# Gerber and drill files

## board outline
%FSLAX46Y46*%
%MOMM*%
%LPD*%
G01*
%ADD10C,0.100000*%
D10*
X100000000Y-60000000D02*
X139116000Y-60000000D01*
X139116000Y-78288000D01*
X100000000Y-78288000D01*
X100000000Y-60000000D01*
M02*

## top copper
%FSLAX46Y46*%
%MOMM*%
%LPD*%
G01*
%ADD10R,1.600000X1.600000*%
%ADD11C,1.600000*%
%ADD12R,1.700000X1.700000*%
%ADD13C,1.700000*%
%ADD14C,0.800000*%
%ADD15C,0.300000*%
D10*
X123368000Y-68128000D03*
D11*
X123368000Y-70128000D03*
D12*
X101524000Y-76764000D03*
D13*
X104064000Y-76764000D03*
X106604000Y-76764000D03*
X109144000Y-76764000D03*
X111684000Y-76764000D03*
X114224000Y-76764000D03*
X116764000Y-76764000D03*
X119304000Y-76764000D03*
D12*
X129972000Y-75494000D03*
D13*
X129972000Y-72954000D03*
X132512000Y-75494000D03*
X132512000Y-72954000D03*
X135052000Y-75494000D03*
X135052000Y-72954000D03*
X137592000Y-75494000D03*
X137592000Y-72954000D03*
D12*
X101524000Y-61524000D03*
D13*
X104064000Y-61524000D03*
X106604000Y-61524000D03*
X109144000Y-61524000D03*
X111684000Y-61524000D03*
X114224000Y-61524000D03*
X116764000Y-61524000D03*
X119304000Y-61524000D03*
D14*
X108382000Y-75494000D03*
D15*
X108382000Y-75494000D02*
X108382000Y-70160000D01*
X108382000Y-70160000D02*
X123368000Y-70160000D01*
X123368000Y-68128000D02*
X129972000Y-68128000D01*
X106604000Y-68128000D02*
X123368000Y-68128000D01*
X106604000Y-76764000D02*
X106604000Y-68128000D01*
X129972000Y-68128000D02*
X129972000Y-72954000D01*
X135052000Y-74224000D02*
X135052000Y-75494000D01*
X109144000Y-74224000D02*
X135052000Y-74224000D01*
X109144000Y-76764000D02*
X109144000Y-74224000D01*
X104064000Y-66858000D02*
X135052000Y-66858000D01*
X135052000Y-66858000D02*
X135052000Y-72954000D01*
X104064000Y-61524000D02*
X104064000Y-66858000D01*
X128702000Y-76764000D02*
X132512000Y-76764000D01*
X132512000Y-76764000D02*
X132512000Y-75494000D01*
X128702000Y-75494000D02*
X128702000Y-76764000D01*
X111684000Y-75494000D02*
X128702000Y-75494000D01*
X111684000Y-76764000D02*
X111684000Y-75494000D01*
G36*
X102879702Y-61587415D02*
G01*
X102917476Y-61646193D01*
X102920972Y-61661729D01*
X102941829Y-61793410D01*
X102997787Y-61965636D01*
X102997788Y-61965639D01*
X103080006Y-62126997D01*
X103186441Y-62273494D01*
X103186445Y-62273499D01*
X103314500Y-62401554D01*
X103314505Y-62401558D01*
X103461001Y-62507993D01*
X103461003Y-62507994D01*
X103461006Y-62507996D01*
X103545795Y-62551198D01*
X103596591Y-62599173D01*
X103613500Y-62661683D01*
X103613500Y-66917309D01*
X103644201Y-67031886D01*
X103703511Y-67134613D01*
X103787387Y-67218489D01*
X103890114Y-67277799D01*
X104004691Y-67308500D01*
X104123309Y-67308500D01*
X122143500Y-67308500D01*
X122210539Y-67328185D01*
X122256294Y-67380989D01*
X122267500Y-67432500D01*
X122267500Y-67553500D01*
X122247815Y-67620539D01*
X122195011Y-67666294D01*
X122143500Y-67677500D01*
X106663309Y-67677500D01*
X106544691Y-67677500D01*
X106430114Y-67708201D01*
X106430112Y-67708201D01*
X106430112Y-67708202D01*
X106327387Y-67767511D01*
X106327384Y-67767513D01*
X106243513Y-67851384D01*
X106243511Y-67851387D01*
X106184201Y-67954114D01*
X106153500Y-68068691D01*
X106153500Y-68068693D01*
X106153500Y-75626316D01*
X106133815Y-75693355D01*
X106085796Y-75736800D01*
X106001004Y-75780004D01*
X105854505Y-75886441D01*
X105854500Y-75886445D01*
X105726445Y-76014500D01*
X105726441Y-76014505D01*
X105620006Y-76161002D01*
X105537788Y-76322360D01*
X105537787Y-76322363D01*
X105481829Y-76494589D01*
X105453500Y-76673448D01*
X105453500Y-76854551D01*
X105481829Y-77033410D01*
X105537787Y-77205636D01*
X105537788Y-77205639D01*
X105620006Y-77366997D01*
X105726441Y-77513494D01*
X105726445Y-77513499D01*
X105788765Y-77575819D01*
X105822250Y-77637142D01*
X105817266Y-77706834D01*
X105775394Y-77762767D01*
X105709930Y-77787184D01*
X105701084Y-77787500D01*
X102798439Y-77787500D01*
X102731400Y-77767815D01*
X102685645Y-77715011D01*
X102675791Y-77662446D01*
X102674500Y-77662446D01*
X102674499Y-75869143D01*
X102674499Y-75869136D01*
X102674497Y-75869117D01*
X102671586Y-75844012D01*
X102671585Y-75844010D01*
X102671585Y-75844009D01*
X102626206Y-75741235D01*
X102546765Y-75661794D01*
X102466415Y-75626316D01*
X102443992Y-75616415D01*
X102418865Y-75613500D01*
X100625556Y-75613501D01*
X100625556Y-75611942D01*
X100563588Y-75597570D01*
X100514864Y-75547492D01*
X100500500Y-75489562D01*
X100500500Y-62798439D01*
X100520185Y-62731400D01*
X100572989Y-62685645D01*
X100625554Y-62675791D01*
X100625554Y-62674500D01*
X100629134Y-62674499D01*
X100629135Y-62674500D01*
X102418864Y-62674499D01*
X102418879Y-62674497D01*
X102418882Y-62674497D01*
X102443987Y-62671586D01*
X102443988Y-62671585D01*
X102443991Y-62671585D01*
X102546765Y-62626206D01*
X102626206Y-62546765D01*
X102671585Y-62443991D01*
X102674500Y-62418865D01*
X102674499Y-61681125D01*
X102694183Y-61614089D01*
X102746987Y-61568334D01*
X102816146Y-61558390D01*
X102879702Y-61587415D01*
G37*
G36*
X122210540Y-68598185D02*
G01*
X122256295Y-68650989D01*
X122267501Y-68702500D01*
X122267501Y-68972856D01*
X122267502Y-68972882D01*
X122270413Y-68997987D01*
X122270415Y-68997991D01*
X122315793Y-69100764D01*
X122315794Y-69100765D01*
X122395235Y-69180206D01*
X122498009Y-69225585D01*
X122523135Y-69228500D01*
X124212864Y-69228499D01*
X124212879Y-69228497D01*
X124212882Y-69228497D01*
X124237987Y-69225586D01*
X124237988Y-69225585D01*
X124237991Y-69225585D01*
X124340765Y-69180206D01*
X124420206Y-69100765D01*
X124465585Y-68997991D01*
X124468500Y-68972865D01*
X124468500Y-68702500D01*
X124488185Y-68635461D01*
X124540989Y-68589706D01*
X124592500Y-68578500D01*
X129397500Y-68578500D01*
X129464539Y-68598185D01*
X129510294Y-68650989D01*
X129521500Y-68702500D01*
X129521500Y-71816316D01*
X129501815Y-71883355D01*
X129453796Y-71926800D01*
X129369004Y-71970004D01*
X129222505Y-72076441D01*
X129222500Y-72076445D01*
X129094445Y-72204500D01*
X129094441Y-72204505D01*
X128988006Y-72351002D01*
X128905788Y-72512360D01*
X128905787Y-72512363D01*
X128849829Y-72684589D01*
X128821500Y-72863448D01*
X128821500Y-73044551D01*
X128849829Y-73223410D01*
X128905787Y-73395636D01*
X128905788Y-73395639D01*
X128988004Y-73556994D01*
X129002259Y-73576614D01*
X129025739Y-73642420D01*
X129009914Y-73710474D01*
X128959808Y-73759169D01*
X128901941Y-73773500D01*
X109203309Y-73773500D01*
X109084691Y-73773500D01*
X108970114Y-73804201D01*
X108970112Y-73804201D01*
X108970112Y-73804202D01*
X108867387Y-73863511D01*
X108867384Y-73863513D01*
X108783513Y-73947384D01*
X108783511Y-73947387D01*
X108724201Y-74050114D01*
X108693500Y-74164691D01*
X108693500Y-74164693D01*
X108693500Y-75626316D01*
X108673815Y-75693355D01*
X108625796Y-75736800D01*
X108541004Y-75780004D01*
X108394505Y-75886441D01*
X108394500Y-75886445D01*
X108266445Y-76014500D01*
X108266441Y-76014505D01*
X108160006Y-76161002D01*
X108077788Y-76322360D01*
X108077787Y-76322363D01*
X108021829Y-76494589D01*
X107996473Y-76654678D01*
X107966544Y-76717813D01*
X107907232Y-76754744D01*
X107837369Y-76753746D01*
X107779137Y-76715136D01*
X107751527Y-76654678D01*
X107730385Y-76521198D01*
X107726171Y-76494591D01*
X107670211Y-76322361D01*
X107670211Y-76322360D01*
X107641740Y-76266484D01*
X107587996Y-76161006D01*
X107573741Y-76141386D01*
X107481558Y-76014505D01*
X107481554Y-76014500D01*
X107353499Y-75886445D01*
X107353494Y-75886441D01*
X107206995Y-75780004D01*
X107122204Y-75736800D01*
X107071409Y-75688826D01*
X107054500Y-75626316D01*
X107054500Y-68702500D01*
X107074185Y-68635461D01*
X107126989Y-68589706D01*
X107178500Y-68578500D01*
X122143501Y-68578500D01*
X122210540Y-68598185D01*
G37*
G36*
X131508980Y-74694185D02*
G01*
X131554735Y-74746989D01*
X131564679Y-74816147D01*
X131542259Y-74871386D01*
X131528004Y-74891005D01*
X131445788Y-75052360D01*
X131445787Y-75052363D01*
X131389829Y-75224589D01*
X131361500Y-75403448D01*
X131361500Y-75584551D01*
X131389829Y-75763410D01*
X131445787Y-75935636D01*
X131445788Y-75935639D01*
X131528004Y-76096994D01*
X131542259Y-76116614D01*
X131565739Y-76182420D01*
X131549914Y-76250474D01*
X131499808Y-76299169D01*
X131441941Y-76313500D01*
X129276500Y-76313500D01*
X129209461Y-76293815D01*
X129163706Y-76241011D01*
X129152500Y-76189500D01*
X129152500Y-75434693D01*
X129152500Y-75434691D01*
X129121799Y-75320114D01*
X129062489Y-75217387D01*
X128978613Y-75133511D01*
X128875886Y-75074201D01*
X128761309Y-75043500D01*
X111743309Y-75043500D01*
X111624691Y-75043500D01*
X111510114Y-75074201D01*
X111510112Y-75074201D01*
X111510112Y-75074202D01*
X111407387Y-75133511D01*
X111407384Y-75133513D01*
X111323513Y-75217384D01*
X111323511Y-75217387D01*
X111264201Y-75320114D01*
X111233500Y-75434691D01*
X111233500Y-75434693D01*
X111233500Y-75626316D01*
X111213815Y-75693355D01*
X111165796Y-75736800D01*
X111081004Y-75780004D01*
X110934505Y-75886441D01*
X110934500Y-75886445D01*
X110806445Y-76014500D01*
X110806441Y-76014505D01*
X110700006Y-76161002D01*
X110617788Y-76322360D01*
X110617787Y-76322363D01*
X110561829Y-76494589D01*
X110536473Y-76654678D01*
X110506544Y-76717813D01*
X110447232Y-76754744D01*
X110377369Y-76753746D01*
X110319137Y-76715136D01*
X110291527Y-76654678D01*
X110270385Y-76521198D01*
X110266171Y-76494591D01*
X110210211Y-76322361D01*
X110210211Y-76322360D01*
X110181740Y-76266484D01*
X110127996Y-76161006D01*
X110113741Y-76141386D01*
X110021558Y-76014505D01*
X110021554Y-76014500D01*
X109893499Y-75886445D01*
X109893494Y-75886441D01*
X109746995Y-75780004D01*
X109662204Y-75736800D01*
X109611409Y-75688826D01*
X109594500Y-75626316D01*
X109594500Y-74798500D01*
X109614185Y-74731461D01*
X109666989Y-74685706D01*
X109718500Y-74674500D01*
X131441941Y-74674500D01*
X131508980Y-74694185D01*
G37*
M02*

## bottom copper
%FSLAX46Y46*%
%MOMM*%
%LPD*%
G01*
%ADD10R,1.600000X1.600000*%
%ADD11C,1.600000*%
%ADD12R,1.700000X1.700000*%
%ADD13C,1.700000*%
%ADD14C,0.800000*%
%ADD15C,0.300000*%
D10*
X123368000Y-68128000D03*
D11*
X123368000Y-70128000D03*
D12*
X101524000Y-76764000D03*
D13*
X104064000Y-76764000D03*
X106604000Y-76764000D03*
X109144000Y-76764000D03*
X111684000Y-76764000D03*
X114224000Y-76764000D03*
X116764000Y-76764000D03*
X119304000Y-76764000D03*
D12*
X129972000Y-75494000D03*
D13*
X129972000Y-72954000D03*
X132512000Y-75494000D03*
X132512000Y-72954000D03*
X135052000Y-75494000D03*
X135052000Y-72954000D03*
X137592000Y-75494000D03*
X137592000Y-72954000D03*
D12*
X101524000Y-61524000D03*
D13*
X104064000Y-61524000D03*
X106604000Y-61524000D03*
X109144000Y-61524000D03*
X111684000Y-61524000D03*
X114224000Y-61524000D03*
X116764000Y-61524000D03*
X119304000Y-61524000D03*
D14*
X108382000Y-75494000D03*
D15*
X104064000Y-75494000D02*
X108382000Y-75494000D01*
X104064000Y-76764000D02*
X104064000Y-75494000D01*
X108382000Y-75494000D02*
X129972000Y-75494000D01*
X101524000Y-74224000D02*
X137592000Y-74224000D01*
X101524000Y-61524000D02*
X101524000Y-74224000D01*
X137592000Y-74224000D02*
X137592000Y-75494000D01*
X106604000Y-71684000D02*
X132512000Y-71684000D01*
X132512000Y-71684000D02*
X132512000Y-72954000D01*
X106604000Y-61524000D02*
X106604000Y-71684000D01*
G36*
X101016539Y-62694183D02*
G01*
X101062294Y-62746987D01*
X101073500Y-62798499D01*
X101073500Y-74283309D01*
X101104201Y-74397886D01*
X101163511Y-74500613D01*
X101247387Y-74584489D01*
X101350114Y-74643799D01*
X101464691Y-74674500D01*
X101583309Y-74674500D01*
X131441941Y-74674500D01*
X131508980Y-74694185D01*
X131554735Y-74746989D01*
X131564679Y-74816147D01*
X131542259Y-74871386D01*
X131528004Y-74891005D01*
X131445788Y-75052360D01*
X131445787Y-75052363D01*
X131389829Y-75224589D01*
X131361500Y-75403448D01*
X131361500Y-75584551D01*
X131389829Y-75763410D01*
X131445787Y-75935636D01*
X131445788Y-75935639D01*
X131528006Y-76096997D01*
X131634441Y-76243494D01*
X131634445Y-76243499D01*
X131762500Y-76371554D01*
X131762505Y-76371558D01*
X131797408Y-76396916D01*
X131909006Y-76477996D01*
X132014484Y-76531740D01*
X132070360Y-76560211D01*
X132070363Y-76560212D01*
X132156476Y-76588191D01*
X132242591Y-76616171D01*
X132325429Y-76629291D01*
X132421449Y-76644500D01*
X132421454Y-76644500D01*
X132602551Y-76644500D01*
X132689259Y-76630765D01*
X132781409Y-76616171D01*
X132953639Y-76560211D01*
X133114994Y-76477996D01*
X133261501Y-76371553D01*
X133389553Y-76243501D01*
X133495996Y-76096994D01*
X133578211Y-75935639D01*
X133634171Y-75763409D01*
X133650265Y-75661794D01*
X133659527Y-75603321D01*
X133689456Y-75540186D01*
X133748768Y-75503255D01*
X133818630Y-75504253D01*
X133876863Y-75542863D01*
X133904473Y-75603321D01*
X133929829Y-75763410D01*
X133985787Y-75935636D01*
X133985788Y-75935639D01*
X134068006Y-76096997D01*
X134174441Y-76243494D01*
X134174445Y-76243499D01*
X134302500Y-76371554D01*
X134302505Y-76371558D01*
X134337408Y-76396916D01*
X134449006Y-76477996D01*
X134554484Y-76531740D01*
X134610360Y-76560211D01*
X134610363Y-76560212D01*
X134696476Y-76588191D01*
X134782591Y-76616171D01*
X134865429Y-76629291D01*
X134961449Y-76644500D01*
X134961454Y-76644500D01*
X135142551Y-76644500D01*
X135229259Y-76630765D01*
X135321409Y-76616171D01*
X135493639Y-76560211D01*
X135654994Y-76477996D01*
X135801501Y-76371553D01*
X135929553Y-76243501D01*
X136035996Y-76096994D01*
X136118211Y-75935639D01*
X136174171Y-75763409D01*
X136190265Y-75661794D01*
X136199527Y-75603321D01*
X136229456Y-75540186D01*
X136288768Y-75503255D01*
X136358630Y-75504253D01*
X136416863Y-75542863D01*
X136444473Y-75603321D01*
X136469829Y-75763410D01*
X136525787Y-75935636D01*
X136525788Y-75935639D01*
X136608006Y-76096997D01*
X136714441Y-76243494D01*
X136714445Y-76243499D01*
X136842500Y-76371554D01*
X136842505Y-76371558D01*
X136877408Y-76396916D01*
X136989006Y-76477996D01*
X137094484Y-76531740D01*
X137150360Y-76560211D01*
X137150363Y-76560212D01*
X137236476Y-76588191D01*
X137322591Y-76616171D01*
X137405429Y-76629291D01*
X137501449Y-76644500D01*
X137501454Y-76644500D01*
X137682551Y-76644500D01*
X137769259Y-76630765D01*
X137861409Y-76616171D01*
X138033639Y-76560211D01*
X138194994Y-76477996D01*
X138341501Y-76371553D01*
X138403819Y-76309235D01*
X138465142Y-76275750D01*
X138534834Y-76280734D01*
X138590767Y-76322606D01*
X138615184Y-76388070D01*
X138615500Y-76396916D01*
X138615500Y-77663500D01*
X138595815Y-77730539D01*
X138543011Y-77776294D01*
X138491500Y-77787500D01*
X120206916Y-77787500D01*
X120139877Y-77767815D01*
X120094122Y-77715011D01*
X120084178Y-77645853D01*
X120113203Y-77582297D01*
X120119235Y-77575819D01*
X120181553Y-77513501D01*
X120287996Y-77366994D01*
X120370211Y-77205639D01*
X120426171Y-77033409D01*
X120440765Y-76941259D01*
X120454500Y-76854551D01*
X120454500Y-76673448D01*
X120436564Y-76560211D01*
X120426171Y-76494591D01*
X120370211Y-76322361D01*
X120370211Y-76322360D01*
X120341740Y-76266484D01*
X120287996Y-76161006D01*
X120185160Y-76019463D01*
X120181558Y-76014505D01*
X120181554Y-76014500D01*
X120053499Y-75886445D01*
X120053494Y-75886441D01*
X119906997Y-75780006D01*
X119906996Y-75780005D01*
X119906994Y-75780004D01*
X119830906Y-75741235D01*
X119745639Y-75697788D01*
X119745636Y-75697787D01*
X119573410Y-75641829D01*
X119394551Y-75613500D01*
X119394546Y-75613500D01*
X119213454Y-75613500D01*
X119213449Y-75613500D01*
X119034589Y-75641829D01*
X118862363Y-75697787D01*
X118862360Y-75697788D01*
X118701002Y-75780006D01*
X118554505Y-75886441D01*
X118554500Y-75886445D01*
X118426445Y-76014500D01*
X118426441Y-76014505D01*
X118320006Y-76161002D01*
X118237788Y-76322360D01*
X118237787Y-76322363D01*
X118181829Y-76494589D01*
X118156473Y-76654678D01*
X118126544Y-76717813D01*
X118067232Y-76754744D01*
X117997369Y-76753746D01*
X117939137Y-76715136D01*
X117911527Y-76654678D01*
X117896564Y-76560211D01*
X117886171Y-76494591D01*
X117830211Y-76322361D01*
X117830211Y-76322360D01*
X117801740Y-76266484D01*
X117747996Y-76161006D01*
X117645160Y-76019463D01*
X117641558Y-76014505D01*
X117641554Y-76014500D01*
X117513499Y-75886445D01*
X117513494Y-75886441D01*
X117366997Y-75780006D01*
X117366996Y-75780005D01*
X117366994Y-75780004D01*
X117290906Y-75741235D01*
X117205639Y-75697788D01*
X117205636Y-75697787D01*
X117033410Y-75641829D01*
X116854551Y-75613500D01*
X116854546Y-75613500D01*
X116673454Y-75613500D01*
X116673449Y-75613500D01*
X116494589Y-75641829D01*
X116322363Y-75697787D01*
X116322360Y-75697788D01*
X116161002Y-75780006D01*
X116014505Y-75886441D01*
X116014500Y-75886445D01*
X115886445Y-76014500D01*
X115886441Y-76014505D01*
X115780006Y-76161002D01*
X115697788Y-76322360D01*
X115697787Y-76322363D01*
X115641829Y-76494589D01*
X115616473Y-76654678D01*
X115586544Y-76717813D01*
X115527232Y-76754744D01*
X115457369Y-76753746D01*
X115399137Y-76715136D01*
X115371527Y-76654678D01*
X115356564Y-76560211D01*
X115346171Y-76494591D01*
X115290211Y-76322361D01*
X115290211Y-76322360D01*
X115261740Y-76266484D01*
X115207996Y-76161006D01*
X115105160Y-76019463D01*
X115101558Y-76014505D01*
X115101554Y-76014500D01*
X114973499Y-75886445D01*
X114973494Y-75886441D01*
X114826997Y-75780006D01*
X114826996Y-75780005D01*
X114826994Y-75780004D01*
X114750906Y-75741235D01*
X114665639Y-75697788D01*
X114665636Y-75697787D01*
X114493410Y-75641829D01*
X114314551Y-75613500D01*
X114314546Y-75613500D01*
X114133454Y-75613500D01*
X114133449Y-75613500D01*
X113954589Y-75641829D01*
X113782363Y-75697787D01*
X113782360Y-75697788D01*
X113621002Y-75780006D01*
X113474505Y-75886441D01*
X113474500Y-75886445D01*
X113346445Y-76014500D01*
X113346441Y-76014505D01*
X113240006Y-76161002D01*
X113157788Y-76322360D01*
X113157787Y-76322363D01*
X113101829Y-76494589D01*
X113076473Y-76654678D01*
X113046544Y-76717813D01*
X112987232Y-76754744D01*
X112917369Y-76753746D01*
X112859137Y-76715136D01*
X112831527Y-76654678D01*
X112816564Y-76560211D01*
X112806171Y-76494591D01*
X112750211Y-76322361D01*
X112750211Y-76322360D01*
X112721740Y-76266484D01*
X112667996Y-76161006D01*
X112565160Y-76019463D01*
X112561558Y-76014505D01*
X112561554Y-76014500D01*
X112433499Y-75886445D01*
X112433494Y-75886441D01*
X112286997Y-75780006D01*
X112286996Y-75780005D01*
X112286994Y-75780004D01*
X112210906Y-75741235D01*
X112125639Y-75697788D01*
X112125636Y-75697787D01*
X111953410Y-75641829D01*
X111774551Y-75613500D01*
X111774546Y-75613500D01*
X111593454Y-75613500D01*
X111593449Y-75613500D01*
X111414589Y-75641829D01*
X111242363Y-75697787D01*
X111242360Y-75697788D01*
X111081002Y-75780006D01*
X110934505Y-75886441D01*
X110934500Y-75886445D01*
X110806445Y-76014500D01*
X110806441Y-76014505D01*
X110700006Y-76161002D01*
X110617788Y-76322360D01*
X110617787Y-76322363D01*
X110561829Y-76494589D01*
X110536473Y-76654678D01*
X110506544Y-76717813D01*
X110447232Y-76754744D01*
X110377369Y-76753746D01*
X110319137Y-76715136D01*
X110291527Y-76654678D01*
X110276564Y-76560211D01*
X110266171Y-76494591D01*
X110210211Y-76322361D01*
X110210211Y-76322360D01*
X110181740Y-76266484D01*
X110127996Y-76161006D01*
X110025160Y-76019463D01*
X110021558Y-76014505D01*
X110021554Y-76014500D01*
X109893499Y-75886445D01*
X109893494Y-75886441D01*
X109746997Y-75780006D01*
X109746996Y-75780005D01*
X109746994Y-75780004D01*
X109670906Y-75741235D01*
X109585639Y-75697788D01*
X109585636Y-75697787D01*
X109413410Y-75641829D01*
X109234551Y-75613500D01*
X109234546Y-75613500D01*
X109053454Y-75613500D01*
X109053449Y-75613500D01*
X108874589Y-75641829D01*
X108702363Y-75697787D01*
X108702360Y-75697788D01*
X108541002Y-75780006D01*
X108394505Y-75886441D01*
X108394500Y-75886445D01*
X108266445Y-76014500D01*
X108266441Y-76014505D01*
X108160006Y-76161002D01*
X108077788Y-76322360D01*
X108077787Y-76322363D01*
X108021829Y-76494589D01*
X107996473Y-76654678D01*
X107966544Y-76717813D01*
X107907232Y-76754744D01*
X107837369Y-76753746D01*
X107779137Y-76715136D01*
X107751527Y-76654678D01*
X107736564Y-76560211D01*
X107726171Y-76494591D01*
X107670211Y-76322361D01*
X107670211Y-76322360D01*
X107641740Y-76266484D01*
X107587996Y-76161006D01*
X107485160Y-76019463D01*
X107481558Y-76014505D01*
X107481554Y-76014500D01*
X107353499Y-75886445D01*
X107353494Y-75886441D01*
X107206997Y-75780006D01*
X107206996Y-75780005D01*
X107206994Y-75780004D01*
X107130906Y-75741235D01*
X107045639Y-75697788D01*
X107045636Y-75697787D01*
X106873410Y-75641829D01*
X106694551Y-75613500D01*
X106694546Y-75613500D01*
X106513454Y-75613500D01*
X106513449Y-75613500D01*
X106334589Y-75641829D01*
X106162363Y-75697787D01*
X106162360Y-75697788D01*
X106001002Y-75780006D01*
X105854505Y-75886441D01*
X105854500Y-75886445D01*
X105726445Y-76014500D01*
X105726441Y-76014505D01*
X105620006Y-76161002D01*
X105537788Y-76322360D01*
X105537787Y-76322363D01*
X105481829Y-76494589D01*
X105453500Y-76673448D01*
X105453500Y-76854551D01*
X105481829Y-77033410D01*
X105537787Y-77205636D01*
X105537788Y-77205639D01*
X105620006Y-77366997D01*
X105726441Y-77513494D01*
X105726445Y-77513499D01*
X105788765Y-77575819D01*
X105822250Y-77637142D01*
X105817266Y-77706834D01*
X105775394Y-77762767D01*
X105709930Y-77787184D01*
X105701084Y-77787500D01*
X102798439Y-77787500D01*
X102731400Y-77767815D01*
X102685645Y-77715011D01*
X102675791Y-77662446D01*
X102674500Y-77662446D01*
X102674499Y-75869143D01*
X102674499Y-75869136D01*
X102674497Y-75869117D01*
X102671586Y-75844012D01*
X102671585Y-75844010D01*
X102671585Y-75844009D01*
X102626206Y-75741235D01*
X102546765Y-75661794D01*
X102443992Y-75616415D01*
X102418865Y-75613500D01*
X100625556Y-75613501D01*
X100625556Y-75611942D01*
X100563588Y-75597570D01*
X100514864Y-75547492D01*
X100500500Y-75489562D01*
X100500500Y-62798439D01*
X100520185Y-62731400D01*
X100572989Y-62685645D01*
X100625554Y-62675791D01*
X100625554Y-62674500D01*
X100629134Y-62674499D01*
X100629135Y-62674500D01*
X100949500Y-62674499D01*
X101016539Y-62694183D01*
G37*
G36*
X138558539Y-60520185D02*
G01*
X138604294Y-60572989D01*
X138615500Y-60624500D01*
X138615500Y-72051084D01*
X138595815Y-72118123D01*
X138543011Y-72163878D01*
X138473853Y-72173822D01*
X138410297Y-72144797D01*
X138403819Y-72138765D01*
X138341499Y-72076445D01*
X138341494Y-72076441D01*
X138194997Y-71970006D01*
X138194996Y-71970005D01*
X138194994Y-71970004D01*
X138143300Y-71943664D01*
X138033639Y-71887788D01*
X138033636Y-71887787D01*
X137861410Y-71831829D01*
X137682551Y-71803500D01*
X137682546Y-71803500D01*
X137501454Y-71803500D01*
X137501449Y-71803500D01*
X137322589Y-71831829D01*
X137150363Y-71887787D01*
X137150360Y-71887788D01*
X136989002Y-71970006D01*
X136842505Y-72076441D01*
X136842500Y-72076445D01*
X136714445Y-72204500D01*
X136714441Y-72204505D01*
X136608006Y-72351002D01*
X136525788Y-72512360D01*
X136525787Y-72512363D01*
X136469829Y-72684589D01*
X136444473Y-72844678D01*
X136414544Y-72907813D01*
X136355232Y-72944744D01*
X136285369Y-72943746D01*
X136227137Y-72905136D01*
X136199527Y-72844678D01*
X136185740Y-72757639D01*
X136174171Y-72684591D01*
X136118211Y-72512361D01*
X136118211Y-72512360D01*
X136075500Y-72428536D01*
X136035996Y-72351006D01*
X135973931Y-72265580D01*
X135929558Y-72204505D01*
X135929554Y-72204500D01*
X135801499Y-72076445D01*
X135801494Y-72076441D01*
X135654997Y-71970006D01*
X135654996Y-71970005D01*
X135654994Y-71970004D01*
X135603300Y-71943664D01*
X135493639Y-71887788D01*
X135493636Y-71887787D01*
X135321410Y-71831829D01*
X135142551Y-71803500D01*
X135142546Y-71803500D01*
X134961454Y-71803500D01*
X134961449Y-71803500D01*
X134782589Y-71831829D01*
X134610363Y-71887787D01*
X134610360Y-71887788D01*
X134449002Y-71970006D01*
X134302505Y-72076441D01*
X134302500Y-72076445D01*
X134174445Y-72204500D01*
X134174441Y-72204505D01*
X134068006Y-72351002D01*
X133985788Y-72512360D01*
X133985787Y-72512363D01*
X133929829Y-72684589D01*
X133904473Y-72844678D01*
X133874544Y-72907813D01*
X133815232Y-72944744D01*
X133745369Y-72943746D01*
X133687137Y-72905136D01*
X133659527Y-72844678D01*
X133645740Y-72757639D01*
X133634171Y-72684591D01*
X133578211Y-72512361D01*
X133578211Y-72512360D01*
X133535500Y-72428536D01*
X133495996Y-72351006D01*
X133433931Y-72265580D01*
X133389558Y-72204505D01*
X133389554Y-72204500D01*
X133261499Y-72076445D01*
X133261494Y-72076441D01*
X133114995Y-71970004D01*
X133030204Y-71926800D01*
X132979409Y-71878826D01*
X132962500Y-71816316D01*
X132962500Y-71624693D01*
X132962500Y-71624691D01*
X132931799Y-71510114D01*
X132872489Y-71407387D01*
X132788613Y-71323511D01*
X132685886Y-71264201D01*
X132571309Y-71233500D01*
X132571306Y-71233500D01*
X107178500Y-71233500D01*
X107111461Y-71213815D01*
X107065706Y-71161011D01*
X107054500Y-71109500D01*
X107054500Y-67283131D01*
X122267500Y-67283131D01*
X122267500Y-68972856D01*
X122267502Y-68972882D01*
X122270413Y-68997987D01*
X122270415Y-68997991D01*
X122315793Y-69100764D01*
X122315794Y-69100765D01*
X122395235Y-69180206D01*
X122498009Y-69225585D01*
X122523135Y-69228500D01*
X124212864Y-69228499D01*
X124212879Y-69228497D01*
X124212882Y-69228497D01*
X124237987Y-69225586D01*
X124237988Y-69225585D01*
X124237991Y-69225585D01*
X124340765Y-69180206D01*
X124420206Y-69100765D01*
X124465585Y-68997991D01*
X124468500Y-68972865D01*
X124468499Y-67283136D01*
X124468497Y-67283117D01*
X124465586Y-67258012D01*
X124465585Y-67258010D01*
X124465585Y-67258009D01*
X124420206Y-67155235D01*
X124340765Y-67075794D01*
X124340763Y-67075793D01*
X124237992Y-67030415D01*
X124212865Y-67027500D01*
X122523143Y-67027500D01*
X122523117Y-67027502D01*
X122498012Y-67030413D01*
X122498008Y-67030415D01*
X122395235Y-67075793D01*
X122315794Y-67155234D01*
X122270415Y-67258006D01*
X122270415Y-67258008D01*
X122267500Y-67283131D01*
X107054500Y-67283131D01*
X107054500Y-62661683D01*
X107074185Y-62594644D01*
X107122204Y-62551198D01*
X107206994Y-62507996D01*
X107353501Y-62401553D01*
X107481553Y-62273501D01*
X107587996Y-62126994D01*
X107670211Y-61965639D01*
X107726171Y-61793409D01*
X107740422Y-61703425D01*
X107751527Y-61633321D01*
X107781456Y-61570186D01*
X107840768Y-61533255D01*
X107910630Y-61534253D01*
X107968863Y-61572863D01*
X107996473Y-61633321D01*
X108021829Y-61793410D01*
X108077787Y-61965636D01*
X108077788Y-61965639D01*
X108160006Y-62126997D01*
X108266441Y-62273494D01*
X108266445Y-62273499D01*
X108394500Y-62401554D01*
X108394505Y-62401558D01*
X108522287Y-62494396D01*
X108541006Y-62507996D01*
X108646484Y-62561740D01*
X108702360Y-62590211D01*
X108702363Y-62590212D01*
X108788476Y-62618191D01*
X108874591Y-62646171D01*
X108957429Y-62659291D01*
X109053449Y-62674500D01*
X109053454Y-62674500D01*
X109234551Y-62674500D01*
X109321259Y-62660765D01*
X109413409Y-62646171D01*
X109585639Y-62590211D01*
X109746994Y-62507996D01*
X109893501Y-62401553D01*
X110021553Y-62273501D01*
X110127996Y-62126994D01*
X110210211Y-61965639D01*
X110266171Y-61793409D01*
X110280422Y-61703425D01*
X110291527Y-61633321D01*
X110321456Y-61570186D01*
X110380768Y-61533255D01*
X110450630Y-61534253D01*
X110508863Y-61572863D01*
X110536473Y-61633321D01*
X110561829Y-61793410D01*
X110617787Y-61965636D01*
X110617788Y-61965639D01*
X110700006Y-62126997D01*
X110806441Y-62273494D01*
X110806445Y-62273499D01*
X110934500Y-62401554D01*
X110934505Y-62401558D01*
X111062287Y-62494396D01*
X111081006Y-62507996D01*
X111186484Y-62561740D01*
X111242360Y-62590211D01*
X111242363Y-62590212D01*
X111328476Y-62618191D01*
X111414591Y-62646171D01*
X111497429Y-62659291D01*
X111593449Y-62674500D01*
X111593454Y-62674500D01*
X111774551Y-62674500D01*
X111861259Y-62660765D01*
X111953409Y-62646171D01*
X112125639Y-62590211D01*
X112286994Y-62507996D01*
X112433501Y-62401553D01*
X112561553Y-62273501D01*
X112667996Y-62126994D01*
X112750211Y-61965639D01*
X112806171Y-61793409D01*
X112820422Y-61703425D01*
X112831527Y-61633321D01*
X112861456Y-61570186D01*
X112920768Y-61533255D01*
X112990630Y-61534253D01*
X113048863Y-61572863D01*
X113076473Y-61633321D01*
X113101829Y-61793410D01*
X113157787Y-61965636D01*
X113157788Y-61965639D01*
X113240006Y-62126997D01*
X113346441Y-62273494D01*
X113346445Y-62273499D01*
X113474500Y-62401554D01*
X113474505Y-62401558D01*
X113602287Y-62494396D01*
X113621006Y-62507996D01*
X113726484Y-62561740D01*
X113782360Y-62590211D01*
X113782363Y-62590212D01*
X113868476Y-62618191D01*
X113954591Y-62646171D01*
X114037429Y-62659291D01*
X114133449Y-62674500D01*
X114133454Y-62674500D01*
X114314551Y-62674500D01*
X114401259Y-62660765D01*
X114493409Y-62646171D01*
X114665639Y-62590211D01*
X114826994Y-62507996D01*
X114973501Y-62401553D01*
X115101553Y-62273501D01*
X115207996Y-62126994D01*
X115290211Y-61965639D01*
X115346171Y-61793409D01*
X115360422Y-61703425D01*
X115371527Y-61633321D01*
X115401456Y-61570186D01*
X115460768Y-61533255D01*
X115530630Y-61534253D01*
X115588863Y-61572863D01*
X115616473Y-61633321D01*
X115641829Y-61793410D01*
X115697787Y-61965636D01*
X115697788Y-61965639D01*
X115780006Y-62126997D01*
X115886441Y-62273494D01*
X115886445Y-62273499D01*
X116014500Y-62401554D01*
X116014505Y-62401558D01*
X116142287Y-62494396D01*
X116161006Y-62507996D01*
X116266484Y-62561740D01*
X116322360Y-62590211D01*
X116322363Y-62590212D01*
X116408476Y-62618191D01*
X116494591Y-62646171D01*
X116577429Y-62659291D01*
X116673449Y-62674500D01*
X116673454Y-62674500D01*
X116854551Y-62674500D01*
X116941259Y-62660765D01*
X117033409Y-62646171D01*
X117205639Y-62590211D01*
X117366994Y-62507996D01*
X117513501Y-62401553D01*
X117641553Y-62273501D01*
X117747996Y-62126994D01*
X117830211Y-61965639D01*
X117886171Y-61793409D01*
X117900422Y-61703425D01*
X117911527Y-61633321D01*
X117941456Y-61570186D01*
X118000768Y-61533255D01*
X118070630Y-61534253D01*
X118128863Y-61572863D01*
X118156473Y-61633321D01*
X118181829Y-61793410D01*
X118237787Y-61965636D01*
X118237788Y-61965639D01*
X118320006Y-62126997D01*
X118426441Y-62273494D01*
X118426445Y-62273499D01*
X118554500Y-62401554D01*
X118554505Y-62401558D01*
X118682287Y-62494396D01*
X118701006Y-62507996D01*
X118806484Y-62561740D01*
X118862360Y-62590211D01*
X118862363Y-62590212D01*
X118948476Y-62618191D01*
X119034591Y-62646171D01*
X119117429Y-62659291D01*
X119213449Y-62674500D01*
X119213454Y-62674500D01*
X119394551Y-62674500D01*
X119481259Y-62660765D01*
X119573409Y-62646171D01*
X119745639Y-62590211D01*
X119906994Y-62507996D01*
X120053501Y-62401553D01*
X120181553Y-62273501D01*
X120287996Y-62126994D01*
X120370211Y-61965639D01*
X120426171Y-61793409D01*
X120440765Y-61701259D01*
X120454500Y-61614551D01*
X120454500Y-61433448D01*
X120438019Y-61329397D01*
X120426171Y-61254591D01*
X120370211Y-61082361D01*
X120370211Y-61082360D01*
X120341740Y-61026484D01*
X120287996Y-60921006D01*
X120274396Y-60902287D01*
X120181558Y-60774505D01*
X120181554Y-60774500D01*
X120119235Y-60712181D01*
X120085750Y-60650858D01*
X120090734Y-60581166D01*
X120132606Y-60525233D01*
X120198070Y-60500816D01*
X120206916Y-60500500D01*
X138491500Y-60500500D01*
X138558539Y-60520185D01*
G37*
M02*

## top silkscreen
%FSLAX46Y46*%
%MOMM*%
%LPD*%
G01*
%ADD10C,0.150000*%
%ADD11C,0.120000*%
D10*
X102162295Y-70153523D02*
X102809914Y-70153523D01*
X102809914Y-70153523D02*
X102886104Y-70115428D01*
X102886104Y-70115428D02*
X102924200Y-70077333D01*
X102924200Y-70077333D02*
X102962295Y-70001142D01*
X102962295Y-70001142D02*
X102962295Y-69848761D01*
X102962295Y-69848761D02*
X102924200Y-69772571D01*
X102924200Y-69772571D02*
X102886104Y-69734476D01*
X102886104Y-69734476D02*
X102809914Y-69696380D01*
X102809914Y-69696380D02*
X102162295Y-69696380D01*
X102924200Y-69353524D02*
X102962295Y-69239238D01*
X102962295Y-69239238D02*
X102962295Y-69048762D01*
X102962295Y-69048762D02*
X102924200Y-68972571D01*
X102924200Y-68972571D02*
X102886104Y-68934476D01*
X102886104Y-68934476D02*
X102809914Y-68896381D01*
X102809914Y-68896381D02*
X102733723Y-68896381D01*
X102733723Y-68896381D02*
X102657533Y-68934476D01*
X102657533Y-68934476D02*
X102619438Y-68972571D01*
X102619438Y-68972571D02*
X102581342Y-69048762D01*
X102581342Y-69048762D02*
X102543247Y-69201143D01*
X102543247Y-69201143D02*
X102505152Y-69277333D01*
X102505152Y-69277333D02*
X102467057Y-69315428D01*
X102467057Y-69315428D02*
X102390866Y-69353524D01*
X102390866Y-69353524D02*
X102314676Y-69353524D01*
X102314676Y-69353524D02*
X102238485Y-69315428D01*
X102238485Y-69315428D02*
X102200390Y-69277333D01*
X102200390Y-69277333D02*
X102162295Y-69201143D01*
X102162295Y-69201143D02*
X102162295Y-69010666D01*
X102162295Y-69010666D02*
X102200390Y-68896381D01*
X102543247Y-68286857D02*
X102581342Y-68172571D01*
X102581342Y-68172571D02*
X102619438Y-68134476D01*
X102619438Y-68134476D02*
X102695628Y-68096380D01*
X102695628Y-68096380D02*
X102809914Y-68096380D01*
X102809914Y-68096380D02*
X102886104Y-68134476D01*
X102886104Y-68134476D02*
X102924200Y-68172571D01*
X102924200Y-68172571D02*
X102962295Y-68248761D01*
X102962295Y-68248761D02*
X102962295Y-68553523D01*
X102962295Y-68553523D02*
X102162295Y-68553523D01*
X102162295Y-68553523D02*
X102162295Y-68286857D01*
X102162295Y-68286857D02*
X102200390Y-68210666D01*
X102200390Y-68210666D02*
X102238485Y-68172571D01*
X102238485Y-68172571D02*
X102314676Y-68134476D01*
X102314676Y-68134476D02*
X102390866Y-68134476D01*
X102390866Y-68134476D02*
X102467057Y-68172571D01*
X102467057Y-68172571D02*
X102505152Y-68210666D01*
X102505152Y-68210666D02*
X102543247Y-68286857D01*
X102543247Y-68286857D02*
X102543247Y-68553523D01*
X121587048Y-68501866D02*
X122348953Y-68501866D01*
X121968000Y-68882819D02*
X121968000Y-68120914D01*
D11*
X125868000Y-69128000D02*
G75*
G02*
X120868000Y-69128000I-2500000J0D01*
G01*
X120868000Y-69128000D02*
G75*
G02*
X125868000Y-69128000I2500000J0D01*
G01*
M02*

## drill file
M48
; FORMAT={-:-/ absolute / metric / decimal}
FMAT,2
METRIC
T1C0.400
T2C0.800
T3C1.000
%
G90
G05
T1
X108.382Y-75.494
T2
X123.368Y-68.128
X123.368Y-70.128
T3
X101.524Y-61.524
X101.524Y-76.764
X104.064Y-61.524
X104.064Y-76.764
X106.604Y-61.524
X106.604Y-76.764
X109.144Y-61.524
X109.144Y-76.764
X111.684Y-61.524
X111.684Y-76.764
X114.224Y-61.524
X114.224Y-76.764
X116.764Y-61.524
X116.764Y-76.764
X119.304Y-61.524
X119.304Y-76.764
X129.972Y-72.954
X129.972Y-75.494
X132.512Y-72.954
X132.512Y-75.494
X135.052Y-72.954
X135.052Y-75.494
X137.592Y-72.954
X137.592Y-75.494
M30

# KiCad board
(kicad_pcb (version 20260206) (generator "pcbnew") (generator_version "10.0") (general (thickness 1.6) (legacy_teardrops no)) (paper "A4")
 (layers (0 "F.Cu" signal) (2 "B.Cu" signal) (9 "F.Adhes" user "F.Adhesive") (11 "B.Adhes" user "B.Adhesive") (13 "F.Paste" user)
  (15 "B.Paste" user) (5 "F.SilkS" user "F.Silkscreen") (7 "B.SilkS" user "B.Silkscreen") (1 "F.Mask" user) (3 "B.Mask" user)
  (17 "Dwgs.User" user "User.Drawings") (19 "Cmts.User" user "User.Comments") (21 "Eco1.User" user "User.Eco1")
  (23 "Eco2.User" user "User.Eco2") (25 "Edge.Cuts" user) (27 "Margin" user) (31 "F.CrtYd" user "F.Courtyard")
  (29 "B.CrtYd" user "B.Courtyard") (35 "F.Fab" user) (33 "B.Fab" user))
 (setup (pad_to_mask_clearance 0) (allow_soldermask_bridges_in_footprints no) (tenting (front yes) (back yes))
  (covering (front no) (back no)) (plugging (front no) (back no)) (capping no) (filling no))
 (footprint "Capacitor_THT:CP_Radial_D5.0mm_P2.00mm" (layer "F.Cu") (at 123.368 68.128)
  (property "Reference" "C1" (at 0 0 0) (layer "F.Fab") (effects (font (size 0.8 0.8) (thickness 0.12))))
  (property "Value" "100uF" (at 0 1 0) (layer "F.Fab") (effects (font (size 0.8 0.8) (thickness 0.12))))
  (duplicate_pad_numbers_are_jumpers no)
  (fp_circle (center 0 1) (end 2.5 1) (stroke (width 0.12) (type solid)) (fill no) (layer "F.SilkS"))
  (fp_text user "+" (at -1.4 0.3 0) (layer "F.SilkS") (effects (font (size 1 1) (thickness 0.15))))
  (pad "1" thru_hole rect (at 0 0) (size 1.6 1.6) (drill 0.8) (layers "*.Cu" "*.Mask") (remove_unused_layers no) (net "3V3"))
  (pad "2" thru_hole circle (at 0 2) (size 1.6 1.6) (drill 0.8) (layers "*.Cu" "*.Mask") (remove_unused_layers no) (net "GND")
   (zone_connect 2)))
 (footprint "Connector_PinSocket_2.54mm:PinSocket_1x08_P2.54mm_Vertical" (layer "F.Cu") (at 101.524 76.764)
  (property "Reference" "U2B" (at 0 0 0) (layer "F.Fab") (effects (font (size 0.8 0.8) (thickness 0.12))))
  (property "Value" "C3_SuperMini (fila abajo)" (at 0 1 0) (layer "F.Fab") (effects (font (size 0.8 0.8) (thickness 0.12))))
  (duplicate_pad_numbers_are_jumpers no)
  (pad "1" thru_hole rect (at 0 0) (size 1.7 1.7) (drill 1) (layers "*.Cu" "*.Mask") (remove_unused_layers no))
  (pad "2" thru_hole circle (at 2.54 0) (size 1.7 1.7) (drill 1) (layers "*.Cu" "*.Mask") (remove_unused_layers no) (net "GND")
   (zone_connect 2))
  (pad "3" thru_hole circle (at 5.08 0) (size 1.7 1.7) (drill 1) (layers "*.Cu" "*.Mask") (remove_unused_layers no) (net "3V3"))
  (pad "4" thru_hole circle (at 7.62 0) (size 1.7 1.7) (drill 1) (layers "*.Cu" "*.Mask") (remove_unused_layers no) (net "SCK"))
  (pad "5" thru_hole circle (at 10.16 0) (size 1.7 1.7) (drill 1) (layers "*.Cu" "*.Mask") (remove_unused_layers no) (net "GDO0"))
  (pad "6" thru_hole circle (at 12.7 0) (size 1.7 1.7) (drill 1) (layers "*.Cu" "*.Mask") (remove_unused_layers no))
  (pad "7" thru_hole circle (at 15.24 0) (size 1.7 1.7) (drill 1) (layers "*.Cu" "*.Mask") (remove_unused_layers no))
  (pad "8" thru_hole circle (at 17.78 0) (size 1.7 1.7) (drill 1) (layers "*.Cu" "*.Mask") (remove_unused_layers no)))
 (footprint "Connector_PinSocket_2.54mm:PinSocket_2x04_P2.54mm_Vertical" (layer "F.Cu") (at 129.972 75.494)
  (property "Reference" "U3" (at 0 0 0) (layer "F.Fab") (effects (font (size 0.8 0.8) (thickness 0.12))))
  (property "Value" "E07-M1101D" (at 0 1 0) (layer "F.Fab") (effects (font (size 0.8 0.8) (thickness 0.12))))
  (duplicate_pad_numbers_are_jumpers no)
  (pad "1" thru_hole rect (at 0 0) (size 1.7 1.7) (drill 1) (layers "*.Cu" "*.Mask") (remove_unused_layers no) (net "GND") (zone_connect 2))
  (pad "2" thru_hole circle (at 0 -2.54) (size 1.7 1.7) (drill 1) (layers "*.Cu" "*.Mask") (remove_unused_layers no) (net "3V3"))
  (pad "3" thru_hole circle (at 2.54 0) (size 1.7 1.7) (drill 1) (layers "*.Cu" "*.Mask") (remove_unused_layers no) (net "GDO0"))
  (pad "4" thru_hole circle (at 2.54 -2.54) (size 1.7 1.7) (drill 1) (layers "*.Cu" "*.Mask") (remove_unused_layers no) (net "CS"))
  (pad "5" thru_hole circle (at 5.08 0) (size 1.7 1.7) (drill 1) (layers "*.Cu" "*.Mask") (remove_unused_layers no) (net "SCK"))
  (pad "6" thru_hole circle (at 5.08 -2.54) (size 1.7 1.7) (drill 1) (layers "*.Cu" "*.Mask") (remove_unused_layers no) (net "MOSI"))
  (pad "7" thru_hole circle (at 7.62 0) (size 1.7 1.7) (drill 1) (layers "*.Cu" "*.Mask") (remove_unused_layers no) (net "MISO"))
  (pad "8" thru_hole circle (at 7.62 -2.54) (size 1.7 1.7) (drill 1) (layers "*.Cu" "*.Mask") (remove_unused_layers no)))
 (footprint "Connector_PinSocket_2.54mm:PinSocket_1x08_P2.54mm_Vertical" (layer "F.Cu") (at 101.524 61.524)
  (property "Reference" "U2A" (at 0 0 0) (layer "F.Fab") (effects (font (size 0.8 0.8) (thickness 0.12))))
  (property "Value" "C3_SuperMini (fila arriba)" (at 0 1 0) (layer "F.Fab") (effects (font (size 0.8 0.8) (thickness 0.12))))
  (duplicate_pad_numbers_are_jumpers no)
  (pad "1" thru_hole rect (at 0 0) (size 1.7 1.7) (drill 1) (layers "*.Cu" "*.Mask") (remove_unused_layers no) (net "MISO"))
  (pad "2" thru_hole circle (at 2.54 0) (size 1.7 1.7) (drill 1) (layers "*.Cu" "*.Mask") (remove_unused_layers no) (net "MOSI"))
  (pad "3" thru_hole circle (at 5.08 0) (size 1.7 1.7) (drill 1) (layers "*.Cu" "*.Mask") (remove_unused_layers no) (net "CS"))
  (pad "4" thru_hole circle (at 7.62 0) (size 1.7 1.7) (drill 1) (layers "*.Cu" "*.Mask") (remove_unused_layers no))
  (pad "5" thru_hole circle (at 10.16 0) (size 1.7 1.7) (drill 1) (layers "*.Cu" "*.Mask") (remove_unused_layers no))
  (pad "6" thru_hole circle (at 12.7 0) (size 1.7 1.7) (drill 1) (layers "*.Cu" "*.Mask") (remove_unused_layers no))
  (pad "7" thru_hole circle (at 15.24 0) (size 1.7 1.7) (drill 1) (layers "*.Cu" "*.Mask") (remove_unused_layers no))
  (pad "8" thru_hole circle (at 17.78 0) (size 1.7 1.7) (drill 1) (layers "*.Cu" "*.Mask") (remove_unused_layers no)))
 (gr_rect (start 100 60) (end 139.116 78.288) (stroke (width 0.1) (type default)) (fill no) (layer "Edge.Cuts"))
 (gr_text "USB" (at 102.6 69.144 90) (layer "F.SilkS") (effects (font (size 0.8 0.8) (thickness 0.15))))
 (segment (start 108.382 75.494) (end 108.382 70.16) (width 0.3) (layer "F.Cu") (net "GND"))
 (segment (start 108.382 70.16) (end 123.368 70.16) (width 0.3) (layer "F.Cu") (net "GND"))
 (via (at 108.382 75.494) (size 0.8) (drill 0.4) (layers "F.Cu" "B.Cu") (capping no) (covering (front no) (back no))
  (plugging (front no) (back no)) (filling no) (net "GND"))
 (segment (start 104.064 75.494) (end 108.382 75.494) (width 0.3) (layer "B.Cu") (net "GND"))
 (segment (start 104.064 76.764) (end 104.064 75.494) (width 0.3) (layer "B.Cu") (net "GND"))
 (segment (start 108.382 75.494) (end 129.972 75.494) (width 0.3) (layer "B.Cu") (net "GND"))
 (segment (start 123.368 68.128) (end 129.972 68.128) (width 0.3) (layer "F.Cu") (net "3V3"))
 (segment (start 106.604 68.128) (end 123.368 68.128) (width 0.3) (layer "F.Cu") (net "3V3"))
 (segment (start 106.604 76.764) (end 106.604 68.128) (width 0.3) (layer "F.Cu") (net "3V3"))
 (segment (start 129.972 68.128) (end 129.972 72.954) (width 0.3) (layer "F.Cu") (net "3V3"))
 (segment (start 135.052 74.224) (end 135.052 75.494) (width 0.3) (layer "F.Cu") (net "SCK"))
 (segment (start 109.144 74.224) (end 135.052 74.224) (width 0.3) (layer "F.Cu") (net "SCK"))
 (segment (start 109.144 76.764) (end 109.144 74.224) (width 0.3) (layer "F.Cu") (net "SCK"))
 (segment (start 101.524 74.224) (end 137.592 74.224) (width 0.3) (layer "B.Cu") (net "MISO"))
 (segment (start 101.524 61.524) (end 101.524 74.224) (width 0.3) (layer "B.Cu") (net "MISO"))
 (segment (start 137.592 74.224) (end 137.592 75.494) (width 0.3) (layer "B.Cu") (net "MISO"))
 (segment (start 104.064 66.858) (end 135.052 66.858) (width 0.3) (layer "F.Cu") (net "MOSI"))
 (segment (start 135.052 66.858) (end 135.052 72.954) (width 0.3) (layer "F.Cu") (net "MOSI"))
 (segment (start 104.064 61.524) (end 104.064 66.858) (width 0.3) (layer "F.Cu") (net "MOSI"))
 (segment (start 106.604 71.684) (end 132.512 71.684) (width 0.3) (layer "B.Cu") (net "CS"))
 (segment (start 132.512 71.684) (end 132.512 72.954) (width 0.3) (layer "B.Cu") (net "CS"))
 (segment (start 106.604 61.524) (end 106.604 71.684) (width 0.3) (layer "B.Cu") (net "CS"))
 (segment (start 128.702 76.764) (end 132.512 76.764) (width 0.3) (layer "F.Cu") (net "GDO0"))
 (segment (start 132.512 76.764) (end 132.512 75.494) (width 0.3) (layer "F.Cu") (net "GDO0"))
 (segment (start 128.702 75.494) (end 128.702 76.764) (width 0.3) (layer "F.Cu") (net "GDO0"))
 (segment (start 111.684 75.494) (end 128.702 75.494) (width 0.3) (layer "F.Cu") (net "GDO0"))
 (segment (start 111.684 76.764) (end 111.684 75.494) (width 0.3) (layer "F.Cu") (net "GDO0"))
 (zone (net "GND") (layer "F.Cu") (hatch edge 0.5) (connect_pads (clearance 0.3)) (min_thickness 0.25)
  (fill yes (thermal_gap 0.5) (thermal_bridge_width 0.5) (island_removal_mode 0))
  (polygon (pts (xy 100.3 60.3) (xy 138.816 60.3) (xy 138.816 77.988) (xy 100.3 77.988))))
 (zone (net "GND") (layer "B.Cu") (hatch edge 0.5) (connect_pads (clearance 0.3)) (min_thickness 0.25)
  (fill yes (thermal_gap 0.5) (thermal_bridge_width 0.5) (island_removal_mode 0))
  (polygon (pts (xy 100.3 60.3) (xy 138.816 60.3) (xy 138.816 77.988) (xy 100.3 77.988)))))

